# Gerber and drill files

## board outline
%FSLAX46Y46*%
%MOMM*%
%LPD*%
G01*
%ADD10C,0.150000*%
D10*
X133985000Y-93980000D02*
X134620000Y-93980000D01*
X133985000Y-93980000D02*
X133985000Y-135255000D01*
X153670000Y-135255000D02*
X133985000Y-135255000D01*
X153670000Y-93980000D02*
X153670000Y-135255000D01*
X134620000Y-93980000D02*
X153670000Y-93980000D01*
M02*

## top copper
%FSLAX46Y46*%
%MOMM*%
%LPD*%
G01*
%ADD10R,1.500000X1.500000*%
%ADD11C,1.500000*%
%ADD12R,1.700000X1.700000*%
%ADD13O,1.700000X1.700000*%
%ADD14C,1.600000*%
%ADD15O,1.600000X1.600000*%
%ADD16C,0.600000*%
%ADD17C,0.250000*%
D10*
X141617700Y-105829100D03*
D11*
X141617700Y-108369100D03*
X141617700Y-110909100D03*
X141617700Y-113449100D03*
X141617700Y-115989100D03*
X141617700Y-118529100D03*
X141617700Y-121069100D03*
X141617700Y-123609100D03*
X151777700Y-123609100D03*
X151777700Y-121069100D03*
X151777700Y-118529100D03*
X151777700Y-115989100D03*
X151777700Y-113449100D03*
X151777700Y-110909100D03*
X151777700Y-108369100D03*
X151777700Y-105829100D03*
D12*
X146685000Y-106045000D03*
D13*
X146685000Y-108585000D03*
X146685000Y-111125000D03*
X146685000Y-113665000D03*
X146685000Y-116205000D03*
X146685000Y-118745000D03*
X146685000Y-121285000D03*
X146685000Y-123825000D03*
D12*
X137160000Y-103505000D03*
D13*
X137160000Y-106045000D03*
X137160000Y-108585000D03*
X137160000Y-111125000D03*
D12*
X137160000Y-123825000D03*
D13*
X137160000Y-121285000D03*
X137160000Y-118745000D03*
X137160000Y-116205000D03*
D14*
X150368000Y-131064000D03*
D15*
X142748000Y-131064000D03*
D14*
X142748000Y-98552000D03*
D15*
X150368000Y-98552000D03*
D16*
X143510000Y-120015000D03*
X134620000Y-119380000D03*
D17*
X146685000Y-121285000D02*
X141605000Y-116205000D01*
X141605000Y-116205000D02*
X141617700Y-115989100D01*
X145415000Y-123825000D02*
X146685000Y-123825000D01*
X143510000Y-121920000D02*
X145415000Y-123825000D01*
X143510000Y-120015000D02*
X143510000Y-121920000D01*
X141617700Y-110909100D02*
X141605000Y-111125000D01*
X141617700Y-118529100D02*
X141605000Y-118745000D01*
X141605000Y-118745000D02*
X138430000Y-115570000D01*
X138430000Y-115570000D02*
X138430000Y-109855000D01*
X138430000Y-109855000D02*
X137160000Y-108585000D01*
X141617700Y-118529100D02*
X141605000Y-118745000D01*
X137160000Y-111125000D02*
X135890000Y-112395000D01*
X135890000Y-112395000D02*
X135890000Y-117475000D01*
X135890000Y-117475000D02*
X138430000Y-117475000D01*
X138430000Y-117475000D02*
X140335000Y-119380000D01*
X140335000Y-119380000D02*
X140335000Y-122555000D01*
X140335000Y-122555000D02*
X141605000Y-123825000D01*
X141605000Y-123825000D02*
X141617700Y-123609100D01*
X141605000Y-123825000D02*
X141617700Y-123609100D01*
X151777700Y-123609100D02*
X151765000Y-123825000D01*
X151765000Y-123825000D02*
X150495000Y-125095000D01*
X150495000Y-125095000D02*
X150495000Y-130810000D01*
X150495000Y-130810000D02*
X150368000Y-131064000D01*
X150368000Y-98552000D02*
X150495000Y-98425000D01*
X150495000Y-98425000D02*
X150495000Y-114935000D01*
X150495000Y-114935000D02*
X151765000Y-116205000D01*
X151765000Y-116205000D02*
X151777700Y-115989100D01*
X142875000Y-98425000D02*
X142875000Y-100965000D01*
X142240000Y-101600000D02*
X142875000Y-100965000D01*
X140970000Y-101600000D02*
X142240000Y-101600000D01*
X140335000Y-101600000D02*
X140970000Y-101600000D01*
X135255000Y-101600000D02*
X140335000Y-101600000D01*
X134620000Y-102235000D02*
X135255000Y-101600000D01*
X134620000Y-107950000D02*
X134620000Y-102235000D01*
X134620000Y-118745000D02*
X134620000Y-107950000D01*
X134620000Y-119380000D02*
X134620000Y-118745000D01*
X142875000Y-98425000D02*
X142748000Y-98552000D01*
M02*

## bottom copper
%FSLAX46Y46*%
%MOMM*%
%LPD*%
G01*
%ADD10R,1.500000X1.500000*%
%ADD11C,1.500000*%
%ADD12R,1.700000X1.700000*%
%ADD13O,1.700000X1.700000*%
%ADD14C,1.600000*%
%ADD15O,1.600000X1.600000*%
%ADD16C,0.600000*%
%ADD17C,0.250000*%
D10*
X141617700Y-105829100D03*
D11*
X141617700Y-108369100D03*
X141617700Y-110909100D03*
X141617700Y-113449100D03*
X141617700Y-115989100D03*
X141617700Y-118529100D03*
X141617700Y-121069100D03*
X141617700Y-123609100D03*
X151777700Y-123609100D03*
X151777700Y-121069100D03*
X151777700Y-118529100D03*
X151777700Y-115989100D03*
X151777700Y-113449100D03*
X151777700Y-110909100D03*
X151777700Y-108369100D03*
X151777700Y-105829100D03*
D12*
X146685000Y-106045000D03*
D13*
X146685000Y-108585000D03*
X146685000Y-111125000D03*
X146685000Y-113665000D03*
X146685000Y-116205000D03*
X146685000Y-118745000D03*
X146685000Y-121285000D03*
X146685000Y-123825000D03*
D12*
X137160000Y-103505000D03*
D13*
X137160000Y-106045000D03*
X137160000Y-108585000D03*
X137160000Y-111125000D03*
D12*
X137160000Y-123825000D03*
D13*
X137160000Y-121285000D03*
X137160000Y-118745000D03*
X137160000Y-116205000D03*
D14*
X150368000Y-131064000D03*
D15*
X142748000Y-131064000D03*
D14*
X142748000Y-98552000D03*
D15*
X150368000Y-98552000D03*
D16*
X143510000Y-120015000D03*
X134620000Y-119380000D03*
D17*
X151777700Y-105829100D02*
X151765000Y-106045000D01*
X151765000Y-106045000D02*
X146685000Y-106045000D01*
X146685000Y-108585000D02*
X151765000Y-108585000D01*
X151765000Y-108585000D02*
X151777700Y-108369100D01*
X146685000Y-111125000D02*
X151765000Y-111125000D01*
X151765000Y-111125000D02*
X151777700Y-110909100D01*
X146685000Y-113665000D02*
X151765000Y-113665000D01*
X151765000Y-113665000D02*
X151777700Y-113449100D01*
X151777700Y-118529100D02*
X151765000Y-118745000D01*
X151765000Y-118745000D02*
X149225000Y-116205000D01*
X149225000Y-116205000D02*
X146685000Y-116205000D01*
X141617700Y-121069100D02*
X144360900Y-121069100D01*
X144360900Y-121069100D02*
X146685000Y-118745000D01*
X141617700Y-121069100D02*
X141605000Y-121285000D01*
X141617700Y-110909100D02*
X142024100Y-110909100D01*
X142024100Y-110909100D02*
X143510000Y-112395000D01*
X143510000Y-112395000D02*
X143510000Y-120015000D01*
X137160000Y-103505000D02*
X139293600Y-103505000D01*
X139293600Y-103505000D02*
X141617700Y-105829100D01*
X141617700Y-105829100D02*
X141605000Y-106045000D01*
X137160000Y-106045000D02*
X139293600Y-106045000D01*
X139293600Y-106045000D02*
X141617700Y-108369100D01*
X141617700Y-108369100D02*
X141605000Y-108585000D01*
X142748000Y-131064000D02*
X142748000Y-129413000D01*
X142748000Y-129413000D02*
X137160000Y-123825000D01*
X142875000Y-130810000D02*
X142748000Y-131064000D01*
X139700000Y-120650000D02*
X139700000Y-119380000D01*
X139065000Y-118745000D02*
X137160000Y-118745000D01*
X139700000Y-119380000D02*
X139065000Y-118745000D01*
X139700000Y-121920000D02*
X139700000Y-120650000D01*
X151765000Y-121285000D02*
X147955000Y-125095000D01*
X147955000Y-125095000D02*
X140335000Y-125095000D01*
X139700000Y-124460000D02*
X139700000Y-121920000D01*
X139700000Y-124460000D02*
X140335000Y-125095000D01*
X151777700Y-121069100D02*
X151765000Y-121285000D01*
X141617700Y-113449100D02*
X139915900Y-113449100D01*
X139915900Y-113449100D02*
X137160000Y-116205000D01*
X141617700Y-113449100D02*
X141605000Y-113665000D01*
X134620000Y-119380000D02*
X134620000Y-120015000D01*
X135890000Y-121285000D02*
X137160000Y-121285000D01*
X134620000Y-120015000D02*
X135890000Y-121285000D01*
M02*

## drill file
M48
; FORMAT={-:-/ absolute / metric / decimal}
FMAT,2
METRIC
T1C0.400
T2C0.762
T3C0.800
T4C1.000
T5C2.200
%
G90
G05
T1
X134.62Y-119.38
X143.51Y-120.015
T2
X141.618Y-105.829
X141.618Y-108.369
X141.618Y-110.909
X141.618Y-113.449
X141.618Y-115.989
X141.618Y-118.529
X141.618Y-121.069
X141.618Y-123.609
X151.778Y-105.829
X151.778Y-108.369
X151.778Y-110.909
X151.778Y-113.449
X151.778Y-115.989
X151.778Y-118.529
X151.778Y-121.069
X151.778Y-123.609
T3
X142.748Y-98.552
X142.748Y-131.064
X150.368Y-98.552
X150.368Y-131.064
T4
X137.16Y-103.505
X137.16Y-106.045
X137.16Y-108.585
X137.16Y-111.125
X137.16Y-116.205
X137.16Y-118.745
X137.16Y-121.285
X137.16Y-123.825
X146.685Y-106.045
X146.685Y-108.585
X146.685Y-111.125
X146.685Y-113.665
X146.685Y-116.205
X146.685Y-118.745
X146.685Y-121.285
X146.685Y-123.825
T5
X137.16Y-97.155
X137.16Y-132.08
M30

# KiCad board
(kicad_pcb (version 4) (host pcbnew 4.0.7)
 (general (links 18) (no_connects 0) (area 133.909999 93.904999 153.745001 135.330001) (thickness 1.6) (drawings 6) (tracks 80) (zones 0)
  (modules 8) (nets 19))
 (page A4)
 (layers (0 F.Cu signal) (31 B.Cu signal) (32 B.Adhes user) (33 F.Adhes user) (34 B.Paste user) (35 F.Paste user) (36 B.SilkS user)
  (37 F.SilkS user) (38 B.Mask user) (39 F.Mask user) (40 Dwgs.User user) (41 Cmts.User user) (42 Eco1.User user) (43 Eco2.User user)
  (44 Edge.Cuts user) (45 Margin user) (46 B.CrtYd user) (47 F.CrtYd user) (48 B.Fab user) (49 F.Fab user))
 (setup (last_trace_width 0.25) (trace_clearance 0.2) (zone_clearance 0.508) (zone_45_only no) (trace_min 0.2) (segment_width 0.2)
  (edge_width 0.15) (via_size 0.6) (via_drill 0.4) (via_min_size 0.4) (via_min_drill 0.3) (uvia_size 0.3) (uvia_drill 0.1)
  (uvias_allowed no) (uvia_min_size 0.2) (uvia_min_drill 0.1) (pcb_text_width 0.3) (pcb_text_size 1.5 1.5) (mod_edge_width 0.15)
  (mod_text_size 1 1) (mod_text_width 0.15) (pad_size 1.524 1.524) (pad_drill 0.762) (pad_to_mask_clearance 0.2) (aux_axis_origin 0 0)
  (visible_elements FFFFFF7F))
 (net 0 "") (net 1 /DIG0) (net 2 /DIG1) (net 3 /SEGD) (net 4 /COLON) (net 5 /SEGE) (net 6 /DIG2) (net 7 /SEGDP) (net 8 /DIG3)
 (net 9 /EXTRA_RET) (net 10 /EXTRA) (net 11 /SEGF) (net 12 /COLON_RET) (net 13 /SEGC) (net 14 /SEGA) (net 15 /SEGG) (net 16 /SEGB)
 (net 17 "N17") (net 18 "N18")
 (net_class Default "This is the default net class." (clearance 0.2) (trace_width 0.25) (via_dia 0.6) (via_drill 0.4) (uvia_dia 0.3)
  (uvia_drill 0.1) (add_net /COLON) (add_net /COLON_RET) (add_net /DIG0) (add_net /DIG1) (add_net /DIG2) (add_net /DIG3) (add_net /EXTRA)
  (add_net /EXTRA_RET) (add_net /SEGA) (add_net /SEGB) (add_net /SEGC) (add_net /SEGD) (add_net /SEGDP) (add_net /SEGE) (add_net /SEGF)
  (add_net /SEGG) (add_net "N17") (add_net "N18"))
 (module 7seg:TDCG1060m (layer F.Cu) (at 140.335 94.615)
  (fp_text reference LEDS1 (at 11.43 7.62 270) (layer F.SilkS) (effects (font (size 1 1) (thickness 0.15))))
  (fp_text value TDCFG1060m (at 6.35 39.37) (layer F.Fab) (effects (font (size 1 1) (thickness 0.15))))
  (pad 1 thru_hole rect (at 1.2827 11.2141) (size 1.5 1.5) (drill 0.762) (layers *.Cu *.Mask) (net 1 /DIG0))
  (pad 2 thru_hole circle (at 1.2827 13.7541) (size 1.5 1.5) (drill 0.762) (layers *.Cu *.Mask) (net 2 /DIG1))
  (pad 3 thru_hole circle (at 1.2827 16.2941) (size 1.5 1.5) (drill 0.762) (layers *.Cu *.Mask) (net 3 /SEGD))
  (pad 4 thru_hole circle (at 1.2827 18.8341) (size 1.5 1.5) (drill 0.762) (layers *.Cu *.Mask) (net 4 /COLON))
  (pad 5 thru_hole circle (at 1.2827 21.3741) (size 1.5 1.5) (drill 0.762) (layers *.Cu *.Mask) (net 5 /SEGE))
  (pad 6 thru_hole circle (at 1.2827 23.9141) (size 1.5 1.5) (drill 0.762) (layers *.Cu *.Mask) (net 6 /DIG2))
  (pad 7 thru_hole circle (at 1.2827 26.4541) (size 1.5 1.5) (drill 0.762) (layers *.Cu *.Mask) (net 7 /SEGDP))
  (pad 8 thru_hole circle (at 1.2827 28.9941) (size 1.5 1.5) (drill 0.762) (layers *.Cu *.Mask) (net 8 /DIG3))
  (pad 9 thru_hole circle (at 11.4427 28.9941) (size 1.5 1.5) (drill 0.762) (layers *.Cu *.Mask) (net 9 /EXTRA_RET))
  (pad 10 thru_hole circle (at 11.4427 26.4541) (size 1.5 1.5) (drill 0.762) (layers *.Cu *.Mask) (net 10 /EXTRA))
  (pad 11 thru_hole circle (at 11.4427 23.9141) (size 1.5 1.5) (drill 0.762) (layers *.Cu *.Mask) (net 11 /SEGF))
  (pad 12 thru_hole circle (at 11.4427 21.3741) (size 1.5 1.5) (drill 0.762) (layers *.Cu *.Mask) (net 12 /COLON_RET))
  (pad 13 thru_hole circle (at 11.4427 18.8341) (size 1.5 1.5) (drill 0.762) (layers *.Cu *.Mask) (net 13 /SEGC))
  (pad 14 thru_hole circle (at 11.4427 16.2941) (size 1.5 1.5) (drill 0.762) (layers *.Cu *.Mask) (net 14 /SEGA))
  (pad 15 thru_hole circle (at 11.4427 13.7541) (size 1.5 1.5) (drill 0.762) (layers *.Cu *.Mask) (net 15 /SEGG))
  (pad 16 thru_hole circle (at 11.4427 11.2141) (size 1.5 1.5) (drill 0.762) (layers *.Cu *.Mask) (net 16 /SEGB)))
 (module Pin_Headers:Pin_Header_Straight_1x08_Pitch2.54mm (layer B.Cu) (at 146.685 106.045 180)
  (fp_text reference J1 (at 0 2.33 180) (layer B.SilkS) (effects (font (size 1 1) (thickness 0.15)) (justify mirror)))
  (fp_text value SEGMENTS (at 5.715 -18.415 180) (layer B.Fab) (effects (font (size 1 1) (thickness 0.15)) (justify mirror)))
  (pad 1 thru_hole rect (at 0 0 180) (size 1.7 1.7) (drill 1) (layers *.Cu *.Mask) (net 16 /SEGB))
  (pad 2 thru_hole oval (at 0 -2.54 180) (size 1.7 1.7) (drill 1) (layers *.Cu *.Mask) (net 15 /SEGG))
  (pad 3 thru_hole oval (at 0 -5.08 180) (size 1.7 1.7) (drill 1) (layers *.Cu *.Mask) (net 14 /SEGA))
  (pad 4 thru_hole oval (at 0 -7.62 180) (size 1.7 1.7) (drill 1) (layers *.Cu *.Mask) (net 13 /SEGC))
  (pad 5 thru_hole oval (at 0 -10.16 180) (size 1.7 1.7) (drill 1) (layers *.Cu *.Mask) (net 11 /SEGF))
  (pad 6 thru_hole oval (at 0 -12.7 180) (size 1.7 1.7) (drill 1) (layers *.Cu *.Mask) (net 7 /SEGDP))
  (pad 7 thru_hole oval (at 0 -15.24 180) (size 1.7 1.7) (drill 1) (layers *.Cu *.Mask) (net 5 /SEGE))
  (pad 8 thru_hole oval (at 0 -17.78 180) (size 1.7 1.7) (drill 1) (layers *.Cu *.Mask) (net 3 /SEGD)))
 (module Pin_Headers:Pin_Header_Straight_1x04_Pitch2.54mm (layer B.Cu) (at 137.16 103.505 180)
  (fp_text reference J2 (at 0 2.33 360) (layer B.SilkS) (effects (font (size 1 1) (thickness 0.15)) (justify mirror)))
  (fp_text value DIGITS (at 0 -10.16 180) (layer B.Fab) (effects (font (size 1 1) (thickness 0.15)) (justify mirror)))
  (pad 1 thru_hole rect (at 0 0 180) (size 1.7 1.7) (drill 1) (layers *.Cu *.Mask) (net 1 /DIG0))
  (pad 2 thru_hole oval (at 0 -2.54 180) (size 1.7 1.7) (drill 1) (layers *.Cu *.Mask) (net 2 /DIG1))
  (pad 3 thru_hole oval (at 0 -5.08 180) (size 1.7 1.7) (drill 1) (layers *.Cu *.Mask) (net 6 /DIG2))
  (pad 4 thru_hole oval (at 0 -7.62 180) (size 1.7 1.7) (drill 1) (layers *.Cu *.Mask) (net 8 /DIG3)))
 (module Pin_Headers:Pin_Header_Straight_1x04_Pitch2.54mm (layer B.Cu) (at 137.16 123.825)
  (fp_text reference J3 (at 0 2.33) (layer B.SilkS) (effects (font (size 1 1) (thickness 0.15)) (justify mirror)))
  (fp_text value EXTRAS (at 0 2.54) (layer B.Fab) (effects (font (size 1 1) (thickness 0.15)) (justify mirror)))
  (pad 1 thru_hole rect (at 0 0) (size 1.7 1.7) (drill 1) (layers *.Cu *.Mask) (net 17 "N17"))
  (pad 2 thru_hole oval (at 0 -2.54) (size 1.7 1.7) (drill 1) (layers *.Cu *.Mask) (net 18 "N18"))
  (pad 3 thru_hole oval (at 0 -5.08) (size 1.7 1.7) (drill 1) (layers *.Cu *.Mask) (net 10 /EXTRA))
  (pad 4 thru_hole oval (at 0 -7.62) (size 1.7 1.7) (drill 1) (layers *.Cu *.Mask) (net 4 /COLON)))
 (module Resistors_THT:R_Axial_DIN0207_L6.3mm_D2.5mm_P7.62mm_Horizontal (layer B.Cu) (at 150.368 131.064 180)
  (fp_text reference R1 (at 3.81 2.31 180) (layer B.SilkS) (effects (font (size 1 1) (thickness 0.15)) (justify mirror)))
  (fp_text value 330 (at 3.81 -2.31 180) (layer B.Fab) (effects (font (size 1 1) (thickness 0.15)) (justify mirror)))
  (pad 1 thru_hole circle (at 0 0 180) (size 1.6 1.6) (drill 0.8) (layers *.Cu *.Mask) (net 9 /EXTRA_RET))
  (pad 2 thru_hole oval (at 7.62 0 180) (size 1.6 1.6) (drill 0.8) (layers *.Cu *.Mask) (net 17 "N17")))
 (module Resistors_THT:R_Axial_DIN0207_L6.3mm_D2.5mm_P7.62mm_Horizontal (layer B.Cu) (at 142.748 98.552)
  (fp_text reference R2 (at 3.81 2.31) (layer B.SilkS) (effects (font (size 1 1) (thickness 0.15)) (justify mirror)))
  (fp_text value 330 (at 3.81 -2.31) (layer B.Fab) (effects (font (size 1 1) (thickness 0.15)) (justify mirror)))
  (pad 1 thru_hole circle (at 0 0) (size 1.6 1.6) (drill 0.8) (layers *.Cu *.Mask) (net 18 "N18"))
  (pad 2 thru_hole oval (at 7.62 0) (size 1.6 1.6) (drill 0.8) (layers *.Cu *.Mask) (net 12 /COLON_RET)))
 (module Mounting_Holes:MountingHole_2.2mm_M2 (layer F.Cu) (at 137.16 132.08)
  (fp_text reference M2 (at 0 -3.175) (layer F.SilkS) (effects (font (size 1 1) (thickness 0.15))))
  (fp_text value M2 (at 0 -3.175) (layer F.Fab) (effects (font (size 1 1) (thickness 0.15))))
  (pad 1 np_thru_hole circle (at 0 0) (size 2.2 2.2) (drill 2.2) (layers *.Cu *.Mask)))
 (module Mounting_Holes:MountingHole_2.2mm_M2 (layer F.Cu) (at 137.16 97.155)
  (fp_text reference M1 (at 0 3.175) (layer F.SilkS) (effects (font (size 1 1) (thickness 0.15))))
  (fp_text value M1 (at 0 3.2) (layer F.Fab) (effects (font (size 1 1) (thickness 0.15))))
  (pad 1 np_thru_hole circle (at 0 0) (size 2.2 2.2) (drill 2.2) (layers *.Cu *.Mask)))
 (gr_line (start 133.985 93.98) (end 134.62 93.98) (angle 90) (layer Edge.Cuts) (width 0.15))
 (gr_line (start 133.985 93.98) (end 133.985 135.255) (angle 90) (layer Edge.Cuts) (width 0.15))
 (gr_line (start 153.67 135.255) (end 133.985 135.255) (angle 90) (layer Edge.Cuts) (width 0.15))
 (gr_line (start 153.67 93.98) (end 153.67 135.255) (angle 90) (layer Edge.Cuts) (width 0.15))
 (gr_line (start 134.62 93.98) (end 153.67 93.98) (angle 90) (layer Edge.Cuts) (width 0.15))
 (segment (start 151.7777 105.8291) (end 151.765 106.045) (width 0.25) (layer B.Cu) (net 16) (status 80000))
 (segment (start 151.765 106.045) (end 146.685 106.045) (width 0.25) (layer B.Cu) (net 16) (status 80000))
 (segment (start 146.685 108.585) (end 151.765 108.585) (width 0.25) (layer B.Cu) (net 15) (status 80000))
 (segment (start 151.765 108.585) (end 151.7777 108.3691) (width 0.25) (layer B.Cu) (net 15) (status 80000))
 (segment (start 146.685 111.125) (end 151.765 111.125) (width 0.25) (layer B.Cu) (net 14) (status 80000))
 (segment (start 151.765 111.125) (end 151.7777 110.9091) (width 0.25) (layer B.Cu) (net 14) (status 80000))
 (segment (start 146.685 113.665) (end 151.765 113.665) (width 0.25) (layer B.Cu) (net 13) (status 80000))
 (segment (start 151.765 113.665) (end 151.7777 113.4491) (width 0.25) (layer B.Cu) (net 13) (status 80000))
 (segment (start 151.7777 118.5291) (end 151.765 118.745) (width 0.25) (layer B.Cu) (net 11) (status 80000))
 (segment (start 151.765 118.745) (end 149.225 116.205) (width 0.25) (layer B.Cu) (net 11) (status 80000))
 (segment (start 149.225 116.205) (end 146.685 116.205) (width 0.25) (layer B.Cu) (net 11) (status 80000))
 (segment (start 141.6177 121.0691) (end 144.3609 121.0691) (width 0.25) (layer B.Cu) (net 7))
 (segment (start 144.3609 121.0691) (end 146.685 118.745) (width 0.25) (layer B.Cu) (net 7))
 (segment (start 141.6177 121.0691) (end 141.605 121.285) (width 0.25) (layer B.Cu) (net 7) (status 80000))
 (segment (start 146.685 121.285) (end 141.605 116.205) (width 0.25) (layer F.Cu) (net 5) (status 80000))
 (segment (start 141.605 116.205) (end 141.6177 115.9891) (width 0.25) (layer F.Cu) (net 5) (status 80000))
 (segment (start 141.6177 110.9091) (end 142.0241 110.9091) (width 0.25) (layer B.Cu) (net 3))
 (segment (start 142.0241 110.9091) (end 143.51 112.395) (width 0.25) (layer B.Cu) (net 3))
 (segment (start 145.415 123.825) (end 146.685 123.825) (width 0.25) (layer F.Cu) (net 3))
 (segment (start 143.51 121.92) (end 145.415 123.825) (width 0.25) (layer F.Cu) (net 3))
 (segment (start 143.51 120.015) (end 143.51 121.92) (width 0.25) (layer F.Cu) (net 3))
 (via (at 143.51 120.015) (size 0.6) (drill 0.4) (layers F.Cu B.Cu) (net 3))
 (segment (start 143.51 112.395) (end 143.51 120.015) (width 0.25) (layer B.Cu) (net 3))
 (segment (start 141.6177 110.9091) (end 141.605 111.125) (width 0.25) (layer F.Cu) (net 3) (status 80000))
 (segment (start 137.16 103.505) (end 139.2936 103.505) (width 0.25) (layer B.Cu) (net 1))
 (segment (start 139.2936 103.505) (end 141.6177 105.8291) (width 0.25) (layer B.Cu) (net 1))
 (segment (start 141.6177 105.8291) (end 141.605 106.045) (width 0.25) (layer B.Cu) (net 1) (status 80000))
 (segment (start 137.16 106.045) (end 139.2936 106.045) (width 0.25) (layer B.Cu) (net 2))
 (segment (start 139.2936 106.045) (end 141.6177 108.3691) (width 0.25) (layer B.Cu) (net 2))
 (segment (start 141.6177 108.3691) (end 141.605 108.585) (width 0.25) (layer B.Cu) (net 2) (status 80000))
 (segment (start 141.6177 118.5291) (end 141.605 118.745) (width 0.25) (layer F.Cu) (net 6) (status 80000))
 (segment (start 141.605 118.745) (end 138.43 115.57) (width 0.25) (layer F.Cu) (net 6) (status 80000))
 (segment (start 138.43 115.57) (end 138.43 109.855) (width 0.25) (layer F.Cu) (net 6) (status 80000))
 (segment (start 138.43 109.855) (end 137.16 108.585) (width 0.25) (layer F.Cu) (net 6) (status 80000))
 (segment (start 141.6177 118.5291) (end 141.605 118.745) (width 0.25) (layer F.Cu) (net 6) (status 80000))
 (segment (start 137.16 111.125) (end 135.89 112.395) (width 0.25) (layer F.Cu) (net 8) (status 80000))
 (segment (start 135.89 112.395) (end 135.89 117.475) (width 0.25) (layer F.Cu) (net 8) (status 80000))
 (segment (start 135.89 117.475) (end 138.43 117.475) (width 0.25) (layer F.Cu) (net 8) (status 80000))
 (segment (start 138.43 117.475) (end 140.335 119.38) (width 0.25) (layer F.Cu) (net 8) (status 80000))
 (segment (start 140.335 119.38) (end 140.335 122.555) (width 0.25) (layer F.Cu) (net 8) (status 80000))
 (segment (start 140.335 122.555) (end 141.605 123.825) (width 0.25) (layer F.Cu) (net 8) (status 80000))
 (segment (start 141.605 123.825) (end 141.6177 123.6091) (width 0.25) (layer F.Cu) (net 8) (status 80000))
 (segment (start 141.605 123.825) (end 141.6177 123.6091) (width 0.25) (layer F.Cu) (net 8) (status 80000))
 (segment (start 142.748 131.064) (end 142.748 129.413) (width 0.25) (layer B.Cu) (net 17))
 (segment (start 142.748 129.413) (end 137.16 123.825) (width 0.25) (layer B.Cu) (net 17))
 (segment (start 142.875 130.81) (end 142.748 131.064) (width 0.25) (layer B.Cu) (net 17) (status 80000))
 (segment (start 139.7 120.65) (end 139.7 119.38) (width 0.25) (layer B.Cu) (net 10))
 (segment (start 139.065 118.745) (end 137.16 118.745) (width 0.25) (layer B.Cu) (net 10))
 (segment (start 139.7 119.38) (end 139.065 118.745) (width 0.25) (layer B.Cu) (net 10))
 (segment (start 139.7 121.92) (end 139.7 120.65) (width 0.25) (layer B.Cu) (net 10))
 (segment (start 151.765 121.285) (end 147.955 125.095) (width 0.25) (layer B.Cu) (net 10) (status 80000))
 (segment (start 147.955 125.095) (end 140.335 125.095) (width 0.25) (layer B.Cu) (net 10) (status 80000))
 (segment (start 139.7 124.46) (end 139.7 121.92) (width 0.25) (layer B.Cu) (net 10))
 (segment (start 139.7 124.46) (end 140.335 125.095) (width 0.25) (layer B.Cu) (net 10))
 (segment (start 151.7777 121.0691) (end 151.765 121.285) (width 0.25) (layer B.Cu) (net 10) (status 80000))
 (segment (start 141.6177 113.4491) (end 139.9159 113.4491) (width 0.25) (layer B.Cu) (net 4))
 (segment (start 139.9159 113.4491) (end 137.16 116.205) (width 0.25) (layer B.Cu) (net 4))
 (segment (start 141.6177 113.4491) (end 141.605 113.665) (width 0.25) (layer B.Cu) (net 4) (status 80000))
 (segment (start 151.7777 123.6091) (end 151.765 123.825) (width 0.25) (layer F.Cu) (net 9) (status 80000))
 (segment (start 151.765 123.825) (end 150.495 125.095) (width 0.25) (layer F.Cu) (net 9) (status 80000))
 (segment (start 150.495 125.095) (end 150.495 130.81) (width 0.25) (layer F.Cu) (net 9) (status 80000))
 (segment (start 150.495 130.81) (end 150.368 131.064) (width 0.25) (layer F.Cu) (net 9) (status 80000))
 (segment (start 150.368 98.552) (end 150.495 98.425) (width 0.25) (layer F.Cu) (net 12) (status 80000))
 (segment (start 150.495 98.425) (end 150.495 114.935) (width 0.25) (layer F.Cu) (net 12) (status 80000))
 (segment (start 150.495 114.935) (end 151.765 116.205) (width 0.25) (layer F.Cu) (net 12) (status 80000))
 (segment (start 151.765 116.205) (end 151.7777 115.9891) (width 0.25) (layer F.Cu) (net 12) (status 80000))
 (segment (start 134.62 119.38) (end 134.62 120.015) (width 0.25) (layer B.Cu) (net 18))
 (segment (start 142.875 98.425) (end 142.875 100.965) (width 0.25) (layer F.Cu) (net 18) (status 80000))
 (segment (start 142.24 101.6) (end 142.875 100.965) (width 0.25) (layer F.Cu) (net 18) (status 80000))
 (segment (start 140.97 101.6) (end 142.24 101.6) (width 0.25) (layer F.Cu) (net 18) (status 80000))
 (segment (start 140.335 101.6) (end 140.97 101.6) (width 0.25) (layer F.Cu) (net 18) (status 80000))
 (segment (start 135.255 101.6) (end 140.335 101.6) (width 0.25) (layer F.Cu) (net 18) (status 80000))
 (segment (start 134.62 102.235) (end 135.255 101.6) (width 0.25) (layer F.Cu) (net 18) (status 80000))
 (segment (start 134.62 107.95) (end 134.62 102.235) (width 0.25) (layer F.Cu) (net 18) (status 80000))
 (segment (start 134.62 118.745) (end 134.62 107.95) (width 0.25) (layer F.Cu) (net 18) (status 80000))
 (segment (start 134.62 119.38) (end 134.62 118.745) (width 0.25) (layer F.Cu) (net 18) (status 80000))
 (via (at 134.62 119.38) (size 0.6) (layers F.Cu B.Cu) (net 18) (status 80000))
 (segment (start 135.89 121.285) (end 137.16 121.285) (width 0.25) (layer B.Cu) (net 18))
 (segment (start 134.62 120.015) (end 135.89 121.285) (width 0.25) (layer B.Cu) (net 18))
 (segment (start 142.875 98.425) (end 142.748 98.552) (width 0.25) (layer F.Cu) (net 18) (status 80000)))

